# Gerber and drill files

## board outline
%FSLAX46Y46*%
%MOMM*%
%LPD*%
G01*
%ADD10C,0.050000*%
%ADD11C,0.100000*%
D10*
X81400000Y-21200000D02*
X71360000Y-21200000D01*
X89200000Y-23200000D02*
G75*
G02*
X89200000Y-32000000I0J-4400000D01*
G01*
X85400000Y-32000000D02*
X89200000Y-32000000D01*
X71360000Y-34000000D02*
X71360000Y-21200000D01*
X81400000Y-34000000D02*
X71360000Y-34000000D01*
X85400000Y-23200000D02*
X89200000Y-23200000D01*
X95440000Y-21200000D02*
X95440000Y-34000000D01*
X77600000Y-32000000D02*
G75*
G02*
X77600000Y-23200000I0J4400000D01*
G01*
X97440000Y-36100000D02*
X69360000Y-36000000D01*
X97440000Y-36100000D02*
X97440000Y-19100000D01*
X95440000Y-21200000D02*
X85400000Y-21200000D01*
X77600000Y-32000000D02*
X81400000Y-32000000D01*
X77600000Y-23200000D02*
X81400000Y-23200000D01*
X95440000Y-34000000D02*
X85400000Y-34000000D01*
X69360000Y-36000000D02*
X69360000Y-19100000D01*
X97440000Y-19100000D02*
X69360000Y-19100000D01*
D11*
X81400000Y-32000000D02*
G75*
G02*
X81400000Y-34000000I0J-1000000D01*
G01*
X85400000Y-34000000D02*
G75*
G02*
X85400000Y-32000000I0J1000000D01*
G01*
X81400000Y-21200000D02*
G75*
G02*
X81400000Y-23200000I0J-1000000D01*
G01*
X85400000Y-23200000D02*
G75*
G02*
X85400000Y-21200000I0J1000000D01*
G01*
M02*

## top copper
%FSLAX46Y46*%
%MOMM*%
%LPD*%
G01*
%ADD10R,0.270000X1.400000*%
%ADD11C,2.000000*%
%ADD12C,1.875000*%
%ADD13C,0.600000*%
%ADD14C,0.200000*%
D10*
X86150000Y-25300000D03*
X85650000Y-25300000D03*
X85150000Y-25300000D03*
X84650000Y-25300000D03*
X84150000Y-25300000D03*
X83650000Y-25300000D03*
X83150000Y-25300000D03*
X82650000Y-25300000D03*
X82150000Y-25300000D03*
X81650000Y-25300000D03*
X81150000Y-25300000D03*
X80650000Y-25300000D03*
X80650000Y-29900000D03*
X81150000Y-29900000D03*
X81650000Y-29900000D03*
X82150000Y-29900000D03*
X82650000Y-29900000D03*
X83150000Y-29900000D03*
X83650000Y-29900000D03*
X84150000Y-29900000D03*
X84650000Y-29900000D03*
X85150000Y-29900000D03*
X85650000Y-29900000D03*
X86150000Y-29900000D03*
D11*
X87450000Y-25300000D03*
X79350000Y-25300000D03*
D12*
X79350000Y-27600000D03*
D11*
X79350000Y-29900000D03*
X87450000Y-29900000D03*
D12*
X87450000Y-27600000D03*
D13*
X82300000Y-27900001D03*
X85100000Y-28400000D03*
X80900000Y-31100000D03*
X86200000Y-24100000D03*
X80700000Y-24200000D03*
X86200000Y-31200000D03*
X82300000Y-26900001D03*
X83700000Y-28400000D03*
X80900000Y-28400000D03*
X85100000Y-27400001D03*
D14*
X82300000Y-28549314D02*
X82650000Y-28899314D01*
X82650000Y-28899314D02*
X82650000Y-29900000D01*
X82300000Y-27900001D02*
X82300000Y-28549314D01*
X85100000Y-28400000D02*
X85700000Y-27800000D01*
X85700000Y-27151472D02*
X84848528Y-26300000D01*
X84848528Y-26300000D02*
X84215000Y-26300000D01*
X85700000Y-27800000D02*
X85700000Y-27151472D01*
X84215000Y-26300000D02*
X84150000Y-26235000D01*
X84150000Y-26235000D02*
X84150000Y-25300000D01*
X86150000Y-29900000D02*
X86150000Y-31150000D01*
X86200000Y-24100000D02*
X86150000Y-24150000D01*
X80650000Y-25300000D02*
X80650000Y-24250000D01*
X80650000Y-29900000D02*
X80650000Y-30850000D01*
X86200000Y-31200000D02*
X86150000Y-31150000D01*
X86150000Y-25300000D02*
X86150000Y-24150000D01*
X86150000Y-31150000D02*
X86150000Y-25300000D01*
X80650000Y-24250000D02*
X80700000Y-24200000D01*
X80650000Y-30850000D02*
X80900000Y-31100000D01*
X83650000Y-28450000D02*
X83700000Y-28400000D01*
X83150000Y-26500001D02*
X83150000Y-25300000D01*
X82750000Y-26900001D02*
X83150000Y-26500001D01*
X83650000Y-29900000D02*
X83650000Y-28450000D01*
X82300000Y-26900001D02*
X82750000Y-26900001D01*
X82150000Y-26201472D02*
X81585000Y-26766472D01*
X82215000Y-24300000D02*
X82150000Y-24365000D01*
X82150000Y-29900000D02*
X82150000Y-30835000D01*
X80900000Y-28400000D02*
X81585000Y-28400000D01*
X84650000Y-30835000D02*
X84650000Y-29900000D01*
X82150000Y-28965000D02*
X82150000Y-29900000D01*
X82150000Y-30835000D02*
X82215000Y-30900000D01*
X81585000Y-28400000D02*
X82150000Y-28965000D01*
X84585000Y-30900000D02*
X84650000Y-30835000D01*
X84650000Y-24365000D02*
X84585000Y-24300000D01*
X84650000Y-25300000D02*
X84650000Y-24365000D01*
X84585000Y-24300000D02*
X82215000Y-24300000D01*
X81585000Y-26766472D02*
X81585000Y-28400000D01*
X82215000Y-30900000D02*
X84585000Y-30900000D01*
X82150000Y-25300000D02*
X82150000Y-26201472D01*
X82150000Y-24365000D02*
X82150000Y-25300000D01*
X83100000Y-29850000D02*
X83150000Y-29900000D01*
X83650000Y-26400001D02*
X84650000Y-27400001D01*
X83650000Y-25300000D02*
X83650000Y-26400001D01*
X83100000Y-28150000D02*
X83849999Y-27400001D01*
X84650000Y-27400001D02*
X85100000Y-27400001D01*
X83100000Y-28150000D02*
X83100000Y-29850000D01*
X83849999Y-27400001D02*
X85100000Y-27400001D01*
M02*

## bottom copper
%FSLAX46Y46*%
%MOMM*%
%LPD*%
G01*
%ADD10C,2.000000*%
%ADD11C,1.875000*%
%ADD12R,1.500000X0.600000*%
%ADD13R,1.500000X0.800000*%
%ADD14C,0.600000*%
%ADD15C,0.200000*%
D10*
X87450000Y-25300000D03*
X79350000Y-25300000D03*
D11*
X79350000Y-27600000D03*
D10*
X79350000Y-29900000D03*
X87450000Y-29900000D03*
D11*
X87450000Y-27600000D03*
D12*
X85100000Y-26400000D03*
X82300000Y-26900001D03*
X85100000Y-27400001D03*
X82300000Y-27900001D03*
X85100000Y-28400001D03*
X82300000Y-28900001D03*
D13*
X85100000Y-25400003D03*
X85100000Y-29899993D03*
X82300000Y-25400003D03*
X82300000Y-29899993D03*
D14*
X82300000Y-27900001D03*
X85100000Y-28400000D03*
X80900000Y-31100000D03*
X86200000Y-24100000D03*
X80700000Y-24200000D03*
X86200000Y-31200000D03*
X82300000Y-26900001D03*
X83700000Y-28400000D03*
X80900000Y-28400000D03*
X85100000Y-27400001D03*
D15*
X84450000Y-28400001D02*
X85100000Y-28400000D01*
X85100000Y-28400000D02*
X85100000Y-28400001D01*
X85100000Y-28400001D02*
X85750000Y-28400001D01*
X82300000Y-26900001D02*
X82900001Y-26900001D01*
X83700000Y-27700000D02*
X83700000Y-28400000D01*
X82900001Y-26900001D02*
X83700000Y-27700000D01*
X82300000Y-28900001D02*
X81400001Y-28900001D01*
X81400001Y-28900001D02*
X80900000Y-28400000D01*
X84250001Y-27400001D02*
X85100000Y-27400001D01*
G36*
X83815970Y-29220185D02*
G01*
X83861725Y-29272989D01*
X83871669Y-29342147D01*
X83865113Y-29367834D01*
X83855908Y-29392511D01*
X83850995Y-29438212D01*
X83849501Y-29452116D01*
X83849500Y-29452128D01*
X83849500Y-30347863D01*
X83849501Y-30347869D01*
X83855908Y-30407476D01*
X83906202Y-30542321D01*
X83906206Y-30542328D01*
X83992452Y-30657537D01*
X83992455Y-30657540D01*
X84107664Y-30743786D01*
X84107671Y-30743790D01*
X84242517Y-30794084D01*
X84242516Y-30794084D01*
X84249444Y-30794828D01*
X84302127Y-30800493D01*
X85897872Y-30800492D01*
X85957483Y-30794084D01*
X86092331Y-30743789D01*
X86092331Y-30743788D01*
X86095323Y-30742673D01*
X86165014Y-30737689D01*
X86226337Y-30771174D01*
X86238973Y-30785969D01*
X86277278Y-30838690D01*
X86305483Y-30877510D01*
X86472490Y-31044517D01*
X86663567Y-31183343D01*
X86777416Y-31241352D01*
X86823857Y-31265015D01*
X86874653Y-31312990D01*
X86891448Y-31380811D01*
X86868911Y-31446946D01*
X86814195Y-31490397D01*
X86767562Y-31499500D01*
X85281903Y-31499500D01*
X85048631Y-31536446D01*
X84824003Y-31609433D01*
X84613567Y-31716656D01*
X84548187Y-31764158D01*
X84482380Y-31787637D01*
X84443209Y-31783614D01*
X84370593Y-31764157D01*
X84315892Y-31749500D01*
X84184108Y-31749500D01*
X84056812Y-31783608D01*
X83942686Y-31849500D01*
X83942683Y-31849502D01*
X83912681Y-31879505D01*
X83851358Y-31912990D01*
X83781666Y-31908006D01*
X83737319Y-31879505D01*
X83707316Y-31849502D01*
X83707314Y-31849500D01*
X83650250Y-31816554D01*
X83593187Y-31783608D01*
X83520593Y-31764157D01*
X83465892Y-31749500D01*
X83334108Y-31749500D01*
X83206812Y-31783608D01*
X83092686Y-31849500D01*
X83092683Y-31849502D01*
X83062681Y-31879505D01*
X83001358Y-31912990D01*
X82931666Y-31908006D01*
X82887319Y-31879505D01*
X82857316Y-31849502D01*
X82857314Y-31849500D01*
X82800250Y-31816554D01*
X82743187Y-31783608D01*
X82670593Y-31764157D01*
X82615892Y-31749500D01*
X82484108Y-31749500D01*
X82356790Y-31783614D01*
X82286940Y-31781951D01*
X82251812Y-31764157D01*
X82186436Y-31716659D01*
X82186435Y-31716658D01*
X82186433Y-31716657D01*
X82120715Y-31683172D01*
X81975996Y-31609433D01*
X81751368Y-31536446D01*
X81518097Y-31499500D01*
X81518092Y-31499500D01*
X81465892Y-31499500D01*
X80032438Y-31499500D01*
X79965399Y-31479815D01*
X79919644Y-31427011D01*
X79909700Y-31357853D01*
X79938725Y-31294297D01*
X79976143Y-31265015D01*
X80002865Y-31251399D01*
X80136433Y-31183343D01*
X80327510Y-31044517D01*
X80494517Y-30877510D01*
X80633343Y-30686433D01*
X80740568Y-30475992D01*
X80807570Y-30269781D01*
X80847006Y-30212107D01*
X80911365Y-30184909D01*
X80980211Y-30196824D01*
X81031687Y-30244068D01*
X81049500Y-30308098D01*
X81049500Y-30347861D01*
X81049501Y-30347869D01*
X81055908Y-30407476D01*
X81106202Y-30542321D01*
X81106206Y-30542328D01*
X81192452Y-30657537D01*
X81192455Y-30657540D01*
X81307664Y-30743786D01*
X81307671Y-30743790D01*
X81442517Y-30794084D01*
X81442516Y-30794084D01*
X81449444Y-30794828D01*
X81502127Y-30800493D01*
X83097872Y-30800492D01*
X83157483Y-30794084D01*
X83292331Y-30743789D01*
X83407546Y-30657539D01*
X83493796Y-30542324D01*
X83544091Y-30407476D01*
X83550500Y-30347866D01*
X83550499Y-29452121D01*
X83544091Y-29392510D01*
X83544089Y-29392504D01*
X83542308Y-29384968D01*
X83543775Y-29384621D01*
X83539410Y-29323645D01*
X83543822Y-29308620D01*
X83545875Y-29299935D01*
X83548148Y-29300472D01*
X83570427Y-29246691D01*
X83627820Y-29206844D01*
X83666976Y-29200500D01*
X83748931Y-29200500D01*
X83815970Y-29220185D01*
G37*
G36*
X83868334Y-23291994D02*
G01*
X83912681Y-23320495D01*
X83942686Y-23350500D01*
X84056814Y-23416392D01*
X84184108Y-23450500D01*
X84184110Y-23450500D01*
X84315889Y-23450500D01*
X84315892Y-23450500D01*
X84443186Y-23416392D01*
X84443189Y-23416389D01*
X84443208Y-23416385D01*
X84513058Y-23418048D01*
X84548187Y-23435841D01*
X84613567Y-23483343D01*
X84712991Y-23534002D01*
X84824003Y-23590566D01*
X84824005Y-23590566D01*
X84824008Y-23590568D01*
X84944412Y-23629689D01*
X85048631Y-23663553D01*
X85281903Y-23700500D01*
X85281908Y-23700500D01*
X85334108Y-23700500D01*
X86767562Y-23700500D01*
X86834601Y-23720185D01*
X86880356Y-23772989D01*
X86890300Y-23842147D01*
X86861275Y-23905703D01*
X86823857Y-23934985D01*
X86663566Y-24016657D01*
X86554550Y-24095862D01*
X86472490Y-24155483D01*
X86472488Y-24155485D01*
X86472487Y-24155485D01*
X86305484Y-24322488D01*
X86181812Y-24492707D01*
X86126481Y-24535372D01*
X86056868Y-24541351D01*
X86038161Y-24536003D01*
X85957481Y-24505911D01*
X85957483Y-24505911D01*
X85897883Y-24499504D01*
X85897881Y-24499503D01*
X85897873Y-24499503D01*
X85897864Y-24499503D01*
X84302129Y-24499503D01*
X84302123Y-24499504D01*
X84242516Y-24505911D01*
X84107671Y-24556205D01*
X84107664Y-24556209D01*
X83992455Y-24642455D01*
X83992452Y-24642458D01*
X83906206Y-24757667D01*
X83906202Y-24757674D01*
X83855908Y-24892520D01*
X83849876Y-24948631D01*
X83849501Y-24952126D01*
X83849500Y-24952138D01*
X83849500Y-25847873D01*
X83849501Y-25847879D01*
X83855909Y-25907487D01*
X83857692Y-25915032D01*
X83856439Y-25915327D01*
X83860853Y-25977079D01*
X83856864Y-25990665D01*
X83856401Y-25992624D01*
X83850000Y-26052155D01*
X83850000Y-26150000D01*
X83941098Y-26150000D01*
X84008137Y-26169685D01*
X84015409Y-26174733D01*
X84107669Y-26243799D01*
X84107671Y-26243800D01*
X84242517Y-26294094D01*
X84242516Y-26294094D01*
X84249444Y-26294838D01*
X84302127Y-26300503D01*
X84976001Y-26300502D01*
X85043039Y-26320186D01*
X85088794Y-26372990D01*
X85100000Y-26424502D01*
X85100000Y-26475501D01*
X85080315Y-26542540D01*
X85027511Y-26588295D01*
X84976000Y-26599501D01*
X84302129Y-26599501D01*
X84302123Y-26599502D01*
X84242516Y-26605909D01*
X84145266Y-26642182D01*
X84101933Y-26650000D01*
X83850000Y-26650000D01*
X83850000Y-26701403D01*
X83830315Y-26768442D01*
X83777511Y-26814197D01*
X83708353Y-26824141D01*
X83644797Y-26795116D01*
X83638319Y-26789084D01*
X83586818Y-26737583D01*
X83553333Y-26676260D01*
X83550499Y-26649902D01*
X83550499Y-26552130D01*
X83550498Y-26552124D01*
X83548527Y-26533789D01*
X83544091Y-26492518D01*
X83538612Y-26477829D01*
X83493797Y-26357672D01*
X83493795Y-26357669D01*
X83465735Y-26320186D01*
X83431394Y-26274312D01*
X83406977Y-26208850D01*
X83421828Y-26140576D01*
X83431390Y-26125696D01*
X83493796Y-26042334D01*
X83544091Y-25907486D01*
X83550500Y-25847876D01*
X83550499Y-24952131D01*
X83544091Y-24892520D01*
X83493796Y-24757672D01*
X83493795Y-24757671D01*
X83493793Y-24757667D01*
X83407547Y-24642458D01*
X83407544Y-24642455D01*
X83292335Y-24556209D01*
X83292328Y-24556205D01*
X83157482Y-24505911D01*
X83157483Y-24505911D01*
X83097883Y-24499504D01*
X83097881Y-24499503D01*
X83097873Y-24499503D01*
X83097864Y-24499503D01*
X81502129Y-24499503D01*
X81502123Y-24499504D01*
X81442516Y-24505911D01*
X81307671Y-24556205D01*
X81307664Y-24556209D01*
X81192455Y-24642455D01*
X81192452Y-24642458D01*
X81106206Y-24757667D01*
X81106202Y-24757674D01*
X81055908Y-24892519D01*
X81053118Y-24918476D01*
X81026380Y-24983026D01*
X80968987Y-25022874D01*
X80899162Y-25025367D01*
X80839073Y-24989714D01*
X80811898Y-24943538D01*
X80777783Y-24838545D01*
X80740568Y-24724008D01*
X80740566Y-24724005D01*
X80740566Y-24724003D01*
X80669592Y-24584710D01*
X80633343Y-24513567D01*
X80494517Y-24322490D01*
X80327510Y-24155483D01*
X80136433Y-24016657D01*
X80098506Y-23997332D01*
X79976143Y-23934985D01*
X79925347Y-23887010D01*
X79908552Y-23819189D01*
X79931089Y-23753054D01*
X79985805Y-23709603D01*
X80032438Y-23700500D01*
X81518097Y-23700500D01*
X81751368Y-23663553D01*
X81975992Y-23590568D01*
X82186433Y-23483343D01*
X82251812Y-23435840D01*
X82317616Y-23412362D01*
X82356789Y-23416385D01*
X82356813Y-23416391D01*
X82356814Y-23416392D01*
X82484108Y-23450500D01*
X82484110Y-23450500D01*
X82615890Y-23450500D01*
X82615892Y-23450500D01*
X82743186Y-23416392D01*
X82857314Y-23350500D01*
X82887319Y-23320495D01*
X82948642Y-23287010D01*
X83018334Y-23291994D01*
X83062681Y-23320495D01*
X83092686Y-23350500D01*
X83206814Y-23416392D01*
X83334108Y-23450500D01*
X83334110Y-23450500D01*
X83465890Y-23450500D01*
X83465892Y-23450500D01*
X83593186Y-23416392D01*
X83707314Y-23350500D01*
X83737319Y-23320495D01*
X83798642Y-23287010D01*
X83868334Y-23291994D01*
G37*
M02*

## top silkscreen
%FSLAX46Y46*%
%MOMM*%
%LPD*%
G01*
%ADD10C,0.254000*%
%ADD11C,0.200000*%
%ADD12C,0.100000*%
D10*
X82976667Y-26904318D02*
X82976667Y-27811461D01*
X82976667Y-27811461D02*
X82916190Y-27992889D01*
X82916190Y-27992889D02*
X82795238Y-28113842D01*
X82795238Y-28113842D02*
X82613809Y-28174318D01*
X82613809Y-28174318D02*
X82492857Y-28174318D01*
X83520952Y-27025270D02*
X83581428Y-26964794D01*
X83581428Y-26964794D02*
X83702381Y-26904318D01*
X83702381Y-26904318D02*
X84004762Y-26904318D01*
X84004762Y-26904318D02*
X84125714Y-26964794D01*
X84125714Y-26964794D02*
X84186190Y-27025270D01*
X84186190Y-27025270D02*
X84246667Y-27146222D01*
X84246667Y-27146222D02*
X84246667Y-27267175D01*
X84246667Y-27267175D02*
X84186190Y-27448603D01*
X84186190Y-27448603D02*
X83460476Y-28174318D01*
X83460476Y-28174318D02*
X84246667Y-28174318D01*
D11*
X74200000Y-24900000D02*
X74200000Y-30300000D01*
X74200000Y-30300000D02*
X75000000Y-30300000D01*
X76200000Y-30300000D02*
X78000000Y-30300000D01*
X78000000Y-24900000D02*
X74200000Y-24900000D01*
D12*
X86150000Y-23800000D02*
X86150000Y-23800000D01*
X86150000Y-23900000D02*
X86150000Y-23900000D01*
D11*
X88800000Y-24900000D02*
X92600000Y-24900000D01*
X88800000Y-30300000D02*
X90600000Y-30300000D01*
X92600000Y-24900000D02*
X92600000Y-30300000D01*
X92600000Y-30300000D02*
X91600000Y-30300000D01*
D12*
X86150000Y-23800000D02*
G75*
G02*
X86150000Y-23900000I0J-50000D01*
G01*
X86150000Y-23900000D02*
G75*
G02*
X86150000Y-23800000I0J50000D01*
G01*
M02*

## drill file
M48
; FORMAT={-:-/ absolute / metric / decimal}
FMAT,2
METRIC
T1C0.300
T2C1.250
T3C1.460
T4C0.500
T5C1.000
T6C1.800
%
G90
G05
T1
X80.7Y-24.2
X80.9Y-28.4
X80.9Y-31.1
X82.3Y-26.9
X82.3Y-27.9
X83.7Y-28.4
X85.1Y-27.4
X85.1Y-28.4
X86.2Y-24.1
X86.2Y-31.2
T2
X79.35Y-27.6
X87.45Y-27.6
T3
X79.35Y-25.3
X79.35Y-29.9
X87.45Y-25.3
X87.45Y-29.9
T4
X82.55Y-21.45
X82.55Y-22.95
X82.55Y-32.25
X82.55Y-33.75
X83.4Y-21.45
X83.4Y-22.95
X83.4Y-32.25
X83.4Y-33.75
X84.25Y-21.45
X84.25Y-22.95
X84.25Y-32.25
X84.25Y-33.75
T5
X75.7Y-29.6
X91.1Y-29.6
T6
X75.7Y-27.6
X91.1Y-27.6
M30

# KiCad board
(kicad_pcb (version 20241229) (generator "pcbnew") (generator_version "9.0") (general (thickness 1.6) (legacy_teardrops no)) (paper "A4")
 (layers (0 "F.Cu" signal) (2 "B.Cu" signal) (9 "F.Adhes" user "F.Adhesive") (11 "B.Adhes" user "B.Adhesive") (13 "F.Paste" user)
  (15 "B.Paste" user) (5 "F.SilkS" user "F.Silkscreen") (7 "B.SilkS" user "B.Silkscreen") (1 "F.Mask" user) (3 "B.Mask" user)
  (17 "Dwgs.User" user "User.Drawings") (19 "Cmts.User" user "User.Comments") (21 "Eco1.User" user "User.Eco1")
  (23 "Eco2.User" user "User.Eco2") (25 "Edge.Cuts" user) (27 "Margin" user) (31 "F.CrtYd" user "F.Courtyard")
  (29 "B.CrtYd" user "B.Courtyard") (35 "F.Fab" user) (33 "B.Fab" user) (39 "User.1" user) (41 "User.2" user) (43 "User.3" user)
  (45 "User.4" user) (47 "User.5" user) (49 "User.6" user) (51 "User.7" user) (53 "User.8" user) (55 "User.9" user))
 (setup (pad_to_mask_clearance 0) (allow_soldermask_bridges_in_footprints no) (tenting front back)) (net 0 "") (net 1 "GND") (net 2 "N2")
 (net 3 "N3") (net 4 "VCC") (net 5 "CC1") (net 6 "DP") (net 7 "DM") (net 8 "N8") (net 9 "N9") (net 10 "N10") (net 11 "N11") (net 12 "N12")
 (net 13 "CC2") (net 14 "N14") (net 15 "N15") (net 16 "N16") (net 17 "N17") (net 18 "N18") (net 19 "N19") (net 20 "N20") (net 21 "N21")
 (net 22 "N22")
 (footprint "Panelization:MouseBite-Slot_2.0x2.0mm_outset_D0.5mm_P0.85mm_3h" (layer "F.Cu") (at 83.4 34)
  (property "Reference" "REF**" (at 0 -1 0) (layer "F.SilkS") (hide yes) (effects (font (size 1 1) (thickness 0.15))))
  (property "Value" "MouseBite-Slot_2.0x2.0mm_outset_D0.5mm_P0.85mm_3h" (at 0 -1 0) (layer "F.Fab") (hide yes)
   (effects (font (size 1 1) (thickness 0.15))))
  (fp_arc (start -2 -2) (mid -1 -1) (end -2 0) (stroke (width 0.1) (type solid)) (layer "Edge.Cuts"))
  (fp_arc (start 2 0) (mid 1 -1) (end 2 -2) (stroke (width 0.1) (type solid)) (layer "Edge.Cuts"))
  (pad "" np_thru_hole circle (at -0.85 -1.75) (size 0.5 0.5) (drill 0.5) (layers "*.Cu" "*.Mask"))
  (pad "" np_thru_hole circle (at -0.85 -0.25 180) (size 0.5 0.5) (drill 0.5) (layers "*.Cu" "*.Mask"))
  (pad "" np_thru_hole circle (at 0 -1.75) (size 0.5 0.5) (drill 0.5) (layers "*.Cu" "*.Mask"))
  (pad "" np_thru_hole circle (at 0 -0.25 180) (size 0.5 0.5) (drill 0.5) (layers "*.Cu" "*.Mask"))
  (pad "" np_thru_hole circle (at 0.85 -1.75) (size 0.5 0.5) (drill 0.5) (layers "*.Cu" "*.Mask"))
  (pad "" np_thru_hole circle (at 0.85 -0.25 180) (size 0.5 0.5) (drill 0.5) (layers "*.Cu" "*.Mask")))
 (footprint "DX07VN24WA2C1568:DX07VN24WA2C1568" (layer "F.Cu") (at 83.4 27.6)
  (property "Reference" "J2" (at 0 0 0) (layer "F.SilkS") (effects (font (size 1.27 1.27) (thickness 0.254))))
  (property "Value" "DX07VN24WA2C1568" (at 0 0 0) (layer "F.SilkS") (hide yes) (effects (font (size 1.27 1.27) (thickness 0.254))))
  (fp_line (start -9.2 -2.7) (end -9.2 2.7) (stroke (width 0.2) (type solid)) (layer "F.SilkS"))
  (fp_line (start -9.2 2.7) (end -8.4 2.7) (stroke (width 0.2) (type solid)) (layer "F.SilkS"))
  (fp_line (start -7.2 2.7) (end -5.4 2.7) (stroke (width 0.2) (type solid)) (layer "F.SilkS"))
  (fp_line (start -5.4 -2.7) (end -9.2 -2.7) (stroke (width 0.2) (type solid)) (layer "F.SilkS"))
  (fp_line (start 2.75 -3.8) (end 2.75 -3.8) (stroke (width 0.1) (type solid)) (layer "F.SilkS"))
  (fp_line (start 2.75 -3.7) (end 2.75 -3.7) (stroke (width 0.1) (type solid)) (layer "F.SilkS"))
  (fp_line (start 5.4 -2.7) (end 9.2 -2.7) (stroke (width 0.2) (type solid)) (layer "F.SilkS"))
  (fp_line (start 5.4 2.7) (end 7.2 2.7) (stroke (width 0.2) (type solid)) (layer "F.SilkS"))
  (fp_line (start 9.2 -2.7) (end 9.2 2.7) (stroke (width 0.2) (type solid)) (layer "F.SilkS"))
  (fp_line (start 9.2 2.7) (end 8.2 2.7) (stroke (width 0.2) (type solid)) (layer "F.SilkS"))
  (fp_arc (start 2.75 -3.8) (mid 2.8 -3.75) (end 2.75 -3.7) (stroke (width 0.1) (type solid)) (layer "F.SilkS"))
  (fp_arc (start 2.75 -3.7) (mid 2.7 -3.75) (end 2.75 -3.8) (stroke (width 0.1) (type solid)) (layer "F.SilkS"))
  (pad "" np_thru_hole circle (at -7.7 0) (size 1.8 1.8) (drill 1.8) (layers "*.Cu" "*.Mask"))
  (pad "" np_thru_hole circle (at -7.7 2) (size 1 1) (drill 1) (layers "*.Cu" "*.Mask"))
  (pad "" np_thru_hole circle (at 7.7 0) (size 1.8 1.8) (drill 1.8) (layers "*.Cu" "*.Mask"))
  (pad "" np_thru_hole circle (at 7.7 2) (size 1 1) (drill 1) (layers "*.Cu" "*.Mask"))
  (pad "A1" smd rect (at 2.75 -2.3) (size 0.27 1.4) (layers "F.Cu" "F.Mask" "F.Paste") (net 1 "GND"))
  (pad "A2" smd rect (at 2.25 -2.3) (size 0.27 1.4) (layers "F.Cu" "F.Mask" "F.Paste") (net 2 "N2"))
  (pad "A3" smd rect (at 1.75 -2.3) (size 0.27 1.4) (layers "F.Cu" "F.Mask" "F.Paste") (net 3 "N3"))
  (pad "A4" smd rect (at 1.25 -2.3) (size 0.27 1.4) (layers "F.Cu" "F.Mask" "F.Paste") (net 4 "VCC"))
  (pad "A5" smd rect (at 0.75 -2.3) (size 0.27 1.4) (layers "F.Cu" "F.Mask" "F.Paste") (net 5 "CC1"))
  (pad "A6" smd rect (at 0.25 -2.3) (size 0.27 1.4) (layers "F.Cu" "F.Mask" "F.Paste") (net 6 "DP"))
  (pad "A7" smd rect (at -0.25 -2.3) (size 0.27 1.4) (layers "F.Cu" "F.Mask" "F.Paste") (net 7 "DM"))
  (pad "A8" smd rect (at -0.75 -2.3) (size 0.27 1.4) (layers "F.Cu" "F.Mask" "F.Paste") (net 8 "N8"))
  (pad "A9" smd rect (at -1.25 -2.3) (size 0.27 1.4) (layers "F.Cu" "F.Mask" "F.Paste") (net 4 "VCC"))
  (pad "A10" smd rect (at -1.75 -2.3) (size 0.27 1.4) (layers "F.Cu" "F.Mask" "F.Paste") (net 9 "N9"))
  (pad "A11" smd rect (at -2.25 -2.3) (size 0.27 1.4) (layers "F.Cu" "F.Mask" "F.Paste") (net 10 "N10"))
  (pad "A12" smd rect (at -2.75 -2.3) (size 0.27 1.4) (layers "F.Cu" "F.Mask" "F.Paste") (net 1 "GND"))
  (pad "B1" smd rect (at -2.75 2.3) (size 0.27 1.4) (layers "F.Cu" "F.Mask" "F.Paste") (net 1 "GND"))
  (pad "B2" smd rect (at -2.25 2.3) (size 0.27 1.4) (layers "F.Cu" "F.Mask" "F.Paste") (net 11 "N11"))
  (pad "B3" smd rect (at -1.75 2.3) (size 0.27 1.4) (layers "F.Cu" "F.Mask" "F.Paste") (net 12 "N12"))
  (pad "B4" smd rect (at -1.25 2.3) (size 0.27 1.4) (layers "F.Cu" "F.Mask" "F.Paste") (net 4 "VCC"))
  (pad "B5" smd rect (at -0.75 2.3) (size 0.27 1.4) (layers "F.Cu" "F.Mask" "F.Paste") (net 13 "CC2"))
  (pad "B6" smd rect (at -0.25 2.3) (size 0.27 1.4) (layers "F.Cu" "F.Mask" "F.Paste") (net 6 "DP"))
  (pad "B7" smd rect (at 0.25 2.3) (size 0.27 1.4) (layers "F.Cu" "F.Mask" "F.Paste") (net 7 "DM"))
  (pad "B8" smd rect (at 0.75 2.3) (size 0.27 1.4) (layers "F.Cu" "F.Mask" "F.Paste") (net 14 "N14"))
  (pad "B9" smd rect (at 1.25 2.3) (size 0.27 1.4) (layers "F.Cu" "F.Mask" "F.Paste") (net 4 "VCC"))
  (pad "B10" smd rect (at 1.75 2.3) (size 0.27 1.4) (layers "F.Cu" "F.Mask" "F.Paste") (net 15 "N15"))
  (pad "B11" smd rect (at 2.25 2.3) (size 0.27 1.4) (layers "F.Cu" "F.Mask" "F.Paste") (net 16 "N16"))
  (pad "B12" smd rect (at 2.75 2.3) (size 0.27 1.4) (layers "F.Cu" "F.Mask" "F.Paste") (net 1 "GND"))
  (pad "MH1" thru_hole circle (at 4.05 -2.3) (size 2 2) (drill 1.46) (layers "*.Cu" "*.Mask") (remove_unused_layers no) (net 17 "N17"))
  (pad "MH2" thru_hole circle (at -4.05 -2.3) (size 2 2) (drill 1.46) (layers "*.Cu" "*.Mask") (remove_unused_layers no) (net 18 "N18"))
  (pad "MH3" thru_hole circle (at -4.05 0) (size 1.875 1.875) (drill 1.25) (layers "*.Cu" "*.Mask") (remove_unused_layers no) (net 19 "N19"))
  (pad "MH4" thru_hole circle (at -4.05 2.3) (size 2 2) (drill 1.46) (layers "*.Cu" "*.Mask") (remove_unused_layers no) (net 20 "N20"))
  (pad "MH5" thru_hole circle (at 4.05 2.3) (size 2 2) (drill 1.46) (layers "*.Cu" "*.Mask") (remove_unused_layers no) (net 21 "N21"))
  (pad "MH6" thru_hole circle (at 4.05 0) (size 1.875 1.875) (drill 1.25) (layers "*.Cu" "*.Mask") (remove_unused_layers no) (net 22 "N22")))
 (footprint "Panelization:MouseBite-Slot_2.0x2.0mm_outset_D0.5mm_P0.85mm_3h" (layer "F.Cu") (at 83.4 23.2)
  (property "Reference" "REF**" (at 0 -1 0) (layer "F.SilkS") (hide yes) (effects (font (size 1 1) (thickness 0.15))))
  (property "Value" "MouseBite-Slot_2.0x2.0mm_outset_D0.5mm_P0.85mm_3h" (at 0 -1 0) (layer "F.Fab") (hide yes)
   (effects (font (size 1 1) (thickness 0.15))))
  (fp_arc (start -2 -2) (mid -1 -1) (end -2 0) (stroke (width 0.1) (type solid)) (layer "Edge.Cuts"))
  (fp_arc (start 2 0) (mid 1 -1) (end 2 -2) (stroke (width 0.1) (type solid)) (layer "Edge.Cuts"))
  (pad "" np_thru_hole circle (at -0.85 -1.75) (size 0.5 0.5) (drill 0.5) (layers "*.Cu" "*.Mask"))
  (pad "" np_thru_hole circle (at -0.85 -0.25 180) (size 0.5 0.5) (drill 0.5) (layers "*.Cu" "*.Mask"))
  (pad "" np_thru_hole circle (at 0 -1.75) (size 0.5 0.5) (drill 0.5) (layers "*.Cu" "*.Mask"))
  (pad "" np_thru_hole circle (at 0 -0.25 180) (size 0.5 0.5) (drill 0.5) (layers "*.Cu" "*.Mask"))
  (pad "" np_thru_hole circle (at 0.85 -1.75) (size 0.5 0.5) (drill 0.5) (layers "*.Cu" "*.Mask"))
  (pad "" np_thru_hole circle (at 0.85 -0.25 180) (size 0.5 0.5) (drill 0.5) (layers "*.Cu" "*.Mask")))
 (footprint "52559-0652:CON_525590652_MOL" (layer "B.Cu") (at 83.7 27.649998 -90)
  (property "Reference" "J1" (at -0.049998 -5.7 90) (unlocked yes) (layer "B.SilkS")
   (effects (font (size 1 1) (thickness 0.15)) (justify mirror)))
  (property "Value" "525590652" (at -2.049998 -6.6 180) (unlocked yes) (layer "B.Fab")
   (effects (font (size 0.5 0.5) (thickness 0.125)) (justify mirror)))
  (pad "1" smd rect (at -1.249998 -1.4 270) (size 0.6 1.5) (layers "B.Cu" "B.Mask" "B.Paste") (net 1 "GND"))
  (pad "2" smd rect (at -0.749997 1.4 270) (size 0.6 1.5) (layers "B.Cu" "B.Mask" "B.Paste") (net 7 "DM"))
  (pad "3" smd rect (at -0.249997 -1.4 270) (size 0.6 1.5) (layers "B.Cu" "B.Mask" "B.Paste") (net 6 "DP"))
  (pad "4" smd rect (at 0.250003 1.4 270) (size 0.6 1.5) (layers "B.Cu" "B.Mask" "B.Paste") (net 13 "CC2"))
  (pad "5" smd rect (at 0.750003 -1.4 270) (size 0.6 1.5) (layers "B.Cu" "B.Mask" "B.Paste") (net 5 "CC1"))
  (pad "6" smd rect (at 1.250003 1.4 270) (size 0.6 1.5) (layers "B.Cu" "B.Mask" "B.Paste") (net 4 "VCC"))
  (pad "P1" smd rect (at -2.249995 -1.4 270) (size 0.8 1.5) (layers "B.Cu" "B.Mask" "B.Paste"))
  (pad "P2" smd rect (at 2.249995 -1.4 270) (size 0.8 1.5) (layers "B.Cu" "B.Mask" "B.Paste"))
  (pad "P3" smd rect (at -2.249995 1.4 270) (size 0.8 1.5) (layers "B.Cu" "B.Mask" "B.Paste"))
  (pad "P4" smd rect (at 2.249995 1.4 270) (size 0.8 1.5) (layers "B.Cu" "B.Mask" "B.Paste")))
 (gr_line (start 81.4 21.2) (end 71.36 21.2) (stroke (width 0.05) (type solid)) (layer "Edge.Cuts"))
 (gr_arc (start 89.2 23.2) (mid 93.6 27.6) (end 89.2 32) (stroke (width 0.05) (type default)) (layer "Edge.Cuts"))
 (gr_line (start 85.4 32) (end 89.2 32) (stroke (width 0.05) (type solid)) (layer "Edge.Cuts"))
 (gr_line (start 71.36 34) (end 71.36 21.2) (stroke (width 0.05) (type default)) (layer "Edge.Cuts"))
 (gr_line (start 81.4 34) (end 71.36 34) (stroke (width 0.05) (type solid)) (layer "Edge.Cuts"))
 (gr_line (start 85.4 23.2) (end 89.2 23.2) (stroke (width 0.05) (type default)) (layer "Edge.Cuts"))
 (gr_line (start 95.44 21.2) (end 95.44 34) (stroke (width 0.05) (type default)) (layer "Edge.Cuts"))
 (gr_arc (start 77.6 32) (mid 73.2 27.6) (end 77.6 23.2) (stroke (width 0.05) (type default)) (layer "Edge.Cuts"))
 (gr_line (start 97.44 36.1) (end 69.36 36) (stroke (width 0.05) (type solid)) (layer "Edge.Cuts"))
 (gr_line (start 97.44 36.1) (end 97.44 19.1) (stroke (width 0.05) (type solid)) (layer "Edge.Cuts"))
 (gr_line (start 95.44 21.2) (end 85.4 21.2) (stroke (width 0.05) (type solid)) (layer "Edge.Cuts"))
 (gr_line (start 77.6 32) (end 81.4 32) (stroke (width 0.05) (type solid)) (layer "Edge.Cuts"))
 (gr_line (start 77.6 23.2) (end 81.4 23.2) (stroke (width 0.05) (type default)) (layer "Edge.Cuts"))
 (gr_line (start 95.44 34) (end 85.4 34) (stroke (width 0.05) (type solid)) (layer "Edge.Cuts"))
 (gr_line (start 69.36 36) (end 69.36 19.1) (stroke (width 0.05) (type solid)) (layer "Edge.Cuts"))
 (gr_line (start 97.44 19.1) (end 69.36 19.1) (stroke (width 0.05) (type solid)) (layer "Edge.Cuts"))
 (segment (start 82.3 28.549314) (end 82.65 28.899314) (width 0.2) (layer "F.Cu") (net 13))
 (segment (start 82.65 28.899314) (end 82.65 29.9) (width 0.2) (layer "F.Cu") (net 13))
 (segment (start 82.3 27.900001) (end 82.3 28.549314) (width 0.2) (layer "F.Cu") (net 13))
 (via (at 82.3 27.900001) (size 0.6) (drill 0.3) (layers "F.Cu" "B.Cu") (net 13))
 (segment (start 85.1 28.4) (end 85.7 27.8) (width 0.2) (layer "F.Cu") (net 5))
 (segment (start 85.7 27.151472) (end 84.848528 26.3) (width 0.2) (layer "F.Cu") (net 5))
 (segment (start 84.848528 26.3) (end 84.215 26.3) (width 0.2) (layer "F.Cu") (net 5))
 (segment (start 85.7 27.8) (end 85.7 27.151472) (width 0.2) (layer "F.Cu") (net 5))
 (segment (start 84.215 26.3) (end 84.15 26.235) (width 0.2) (layer "F.Cu") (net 5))
 (segment (start 84.15 26.235) (end 84.15 25.3) (width 0.2) (layer "F.Cu") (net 5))
 (via (at 85.1 28.4) (size 0.6) (drill 0.3) (layers "F.Cu" "B.Cu") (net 5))
 (segment (start 84.45 28.400001) (end 85.1 28.4) (width 0.2) (layer "B.Cu") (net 5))
 (segment (start 85.1 28.4) (end 85.1 28.400001) (width 0.2) (layer "B.Cu") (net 5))
 (segment (start 85.1 28.400001) (end 85.75 28.400001) (width 0.2) (layer "B.Cu") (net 5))
 (segment (start 86.15 29.9) (end 86.15 31.15) (width 0.2) (layer "F.Cu") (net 1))
 (segment (start 86.2 24.1) (end 86.15 24.15) (width 0.2) (layer "F.Cu") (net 1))
 (segment (start 80.65 25.3) (end 80.65 24.25) (width 0.2) (layer "F.Cu") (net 1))
 (segment (start 80.65 29.9) (end 80.65 30.85) (width 0.2) (layer "F.Cu") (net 1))
 (segment (start 86.2 31.2) (end 86.15 31.15) (width 0.2) (layer "F.Cu") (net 1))
 (segment (start 86.15 25.3) (end 86.15 24.15) (width 0.2) (layer "F.Cu") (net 1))
 (segment (start 86.15 31.15) (end 86.15 25.3) (width 0.2) (layer "F.Cu") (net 1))
 (segment (start 80.65 24.25) (end 80.7 24.2) (width 0.2) (layer "F.Cu") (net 1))
 (segment (start 80.65 30.85) (end 80.9 31.1) (width 0.2) (layer "F.Cu") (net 1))
 (via (at 80.9 31.1) (size 0.6) (drill 0.3) (layers "F.Cu" "B.Cu") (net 1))
 (via (at 86.2 24.1) (size 0.6) (drill 0.3) (layers "F.Cu" "B.Cu") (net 1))
 (via (at 80.7 24.2) (size 0.6) (drill 0.3) (layers "F.Cu" "B.Cu") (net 1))
 (via (at 86.2 31.2) (size 0.6) (drill 0.3) (layers "F.Cu" "B.Cu") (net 1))
 (segment (start 83.65 28.45) (end 83.7 28.4) (width 0.2) (layer "F.Cu") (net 7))
 (segment (start 83.15 26.500001) (end 83.15 25.3) (width 0.2) (layer "F.Cu") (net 7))
 (segment (start 82.75 26.900001) (end 83.15 26.500001) (width 0.2) (layer "F.Cu") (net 7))
 (segment (start 83.65 29.9) (end 83.65 28.45) (width 0.2) (layer "F.Cu") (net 7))
 (segment (start 82.3 26.900001) (end 82.75 26.900001) (width 0.2) (layer "F.Cu") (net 7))
 (via (at 82.3 26.900001) (size 0.6) (drill 0.3) (layers "F.Cu" "B.Cu") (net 7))
 (via (at 83.7 28.4) (size 0.6) (drill 0.3) (layers "F.Cu" "B.Cu") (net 7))
 (segment (start 82.3 26.900001) (end 82.900001 26.900001) (width 0.2) (layer "B.Cu") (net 7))
 (segment (start 83.7 27.7) (end 83.7 28.4) (width 0.2) (layer "B.Cu") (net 7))
 (segment (start 82.900001 26.900001) (end 83.7 27.7) (width 0.2) (layer "B.Cu") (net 7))
 (segment (start 82.15 26.201472) (end 81.585 26.766472) (width 0.2) (layer "F.Cu") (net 4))
 (segment (start 82.215 24.3) (end 82.15 24.365) (width 0.2) (layer "F.Cu") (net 4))
 (segment (start 82.15 29.9) (end 82.15 30.835) (width 0.2) (layer "F.Cu") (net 4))
 (segment (start 80.9 28.4) (end 81.585 28.4) (width 0.2) (layer "F.Cu") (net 4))
 (segment (start 84.65 30.835) (end 84.65 29.9) (width 0.2) (layer "F.Cu") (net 4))
 (segment (start 82.15 28.965) (end 82.15 29.9) (width 0.2) (layer "F.Cu") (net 4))
 (segment (start 82.15 30.835) (end 82.215 30.9) (width 0.2) (layer "F.Cu") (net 4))
 (segment (start 81.585 28.4) (end 82.15 28.965) (width 0.2) (layer "F.Cu") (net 4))
 (segment (start 84.585 30.9) (end 84.65 30.835) (width 0.2) (layer "F.Cu") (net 4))
 (segment (start 84.65 24.365) (end 84.585 24.3) (width 0.2) (layer "F.Cu") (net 4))
 (segment (start 84.65 25.3) (end 84.65 24.365) (width 0.2) (layer "F.Cu") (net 4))
 (segment (start 84.585 24.3) (end 82.215 24.3) (width 0.2) (layer "F.Cu") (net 4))
 (segment (start 81.585 26.766472) (end 81.585 28.4) (width 0.2) (layer "F.Cu") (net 4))
 (segment (start 82.215 30.9) (end 84.585 30.9) (width 0.2) (layer "F.Cu") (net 4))
 (segment (start 82.15 25.3) (end 82.15 26.201472) (width 0.2) (layer "F.Cu") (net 4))
 (segment (start 82.15 24.365) (end 82.15 25.3) (width 0.2) (layer "F.Cu") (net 4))
 (via (at 80.9 28.4) (size 0.6) (drill 0.3) (layers "F.Cu" "B.Cu") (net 4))
 (segment (start 82.3 28.900001) (end 81.400001 28.900001) (width 0.2) (layer "B.Cu") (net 4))
 (segment (start 81.400001 28.900001) (end 80.9 28.4) (width 0.2) (layer "B.Cu") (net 4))
 (segment (start 83.1 29.85) (end 83.15 29.9) (width 0.2) (layer "F.Cu") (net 6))
 (segment (start 83.65 26.400001) (end 84.65 27.400001) (width 0.2) (layer "F.Cu") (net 6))
 (segment (start 83.65 25.3) (end 83.65 26.400001) (width 0.2) (layer "F.Cu") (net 6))
 (segment (start 83.1 28.15) (end 83.849999 27.400001) (width 0.2) (layer "F.Cu") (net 6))
 (segment (start 84.65 27.400001) (end 85.1 27.400001) (width 0.2) (layer "F.Cu") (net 6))
 (segment (start 83.1 28.15) (end 83.1 29.85) (width 0.2) (layer "F.Cu") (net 6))
 (segment (start 83.849999 27.400001) (end 85.1 27.400001) (width 0.2) (layer "F.Cu") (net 6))
 (via (at 85.1 27.400001) (size 0.6) (drill 0.3) (layers "F.Cu" "B.Cu") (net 6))
 (segment (start 84.250001 27.400001) (end 85.1 27.400001) (width 0.2) (layer "B.Cu") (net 6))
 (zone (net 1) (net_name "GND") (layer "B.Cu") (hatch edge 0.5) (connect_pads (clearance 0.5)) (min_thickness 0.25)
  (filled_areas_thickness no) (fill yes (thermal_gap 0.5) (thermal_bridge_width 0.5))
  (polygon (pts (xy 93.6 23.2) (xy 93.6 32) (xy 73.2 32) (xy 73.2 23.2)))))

